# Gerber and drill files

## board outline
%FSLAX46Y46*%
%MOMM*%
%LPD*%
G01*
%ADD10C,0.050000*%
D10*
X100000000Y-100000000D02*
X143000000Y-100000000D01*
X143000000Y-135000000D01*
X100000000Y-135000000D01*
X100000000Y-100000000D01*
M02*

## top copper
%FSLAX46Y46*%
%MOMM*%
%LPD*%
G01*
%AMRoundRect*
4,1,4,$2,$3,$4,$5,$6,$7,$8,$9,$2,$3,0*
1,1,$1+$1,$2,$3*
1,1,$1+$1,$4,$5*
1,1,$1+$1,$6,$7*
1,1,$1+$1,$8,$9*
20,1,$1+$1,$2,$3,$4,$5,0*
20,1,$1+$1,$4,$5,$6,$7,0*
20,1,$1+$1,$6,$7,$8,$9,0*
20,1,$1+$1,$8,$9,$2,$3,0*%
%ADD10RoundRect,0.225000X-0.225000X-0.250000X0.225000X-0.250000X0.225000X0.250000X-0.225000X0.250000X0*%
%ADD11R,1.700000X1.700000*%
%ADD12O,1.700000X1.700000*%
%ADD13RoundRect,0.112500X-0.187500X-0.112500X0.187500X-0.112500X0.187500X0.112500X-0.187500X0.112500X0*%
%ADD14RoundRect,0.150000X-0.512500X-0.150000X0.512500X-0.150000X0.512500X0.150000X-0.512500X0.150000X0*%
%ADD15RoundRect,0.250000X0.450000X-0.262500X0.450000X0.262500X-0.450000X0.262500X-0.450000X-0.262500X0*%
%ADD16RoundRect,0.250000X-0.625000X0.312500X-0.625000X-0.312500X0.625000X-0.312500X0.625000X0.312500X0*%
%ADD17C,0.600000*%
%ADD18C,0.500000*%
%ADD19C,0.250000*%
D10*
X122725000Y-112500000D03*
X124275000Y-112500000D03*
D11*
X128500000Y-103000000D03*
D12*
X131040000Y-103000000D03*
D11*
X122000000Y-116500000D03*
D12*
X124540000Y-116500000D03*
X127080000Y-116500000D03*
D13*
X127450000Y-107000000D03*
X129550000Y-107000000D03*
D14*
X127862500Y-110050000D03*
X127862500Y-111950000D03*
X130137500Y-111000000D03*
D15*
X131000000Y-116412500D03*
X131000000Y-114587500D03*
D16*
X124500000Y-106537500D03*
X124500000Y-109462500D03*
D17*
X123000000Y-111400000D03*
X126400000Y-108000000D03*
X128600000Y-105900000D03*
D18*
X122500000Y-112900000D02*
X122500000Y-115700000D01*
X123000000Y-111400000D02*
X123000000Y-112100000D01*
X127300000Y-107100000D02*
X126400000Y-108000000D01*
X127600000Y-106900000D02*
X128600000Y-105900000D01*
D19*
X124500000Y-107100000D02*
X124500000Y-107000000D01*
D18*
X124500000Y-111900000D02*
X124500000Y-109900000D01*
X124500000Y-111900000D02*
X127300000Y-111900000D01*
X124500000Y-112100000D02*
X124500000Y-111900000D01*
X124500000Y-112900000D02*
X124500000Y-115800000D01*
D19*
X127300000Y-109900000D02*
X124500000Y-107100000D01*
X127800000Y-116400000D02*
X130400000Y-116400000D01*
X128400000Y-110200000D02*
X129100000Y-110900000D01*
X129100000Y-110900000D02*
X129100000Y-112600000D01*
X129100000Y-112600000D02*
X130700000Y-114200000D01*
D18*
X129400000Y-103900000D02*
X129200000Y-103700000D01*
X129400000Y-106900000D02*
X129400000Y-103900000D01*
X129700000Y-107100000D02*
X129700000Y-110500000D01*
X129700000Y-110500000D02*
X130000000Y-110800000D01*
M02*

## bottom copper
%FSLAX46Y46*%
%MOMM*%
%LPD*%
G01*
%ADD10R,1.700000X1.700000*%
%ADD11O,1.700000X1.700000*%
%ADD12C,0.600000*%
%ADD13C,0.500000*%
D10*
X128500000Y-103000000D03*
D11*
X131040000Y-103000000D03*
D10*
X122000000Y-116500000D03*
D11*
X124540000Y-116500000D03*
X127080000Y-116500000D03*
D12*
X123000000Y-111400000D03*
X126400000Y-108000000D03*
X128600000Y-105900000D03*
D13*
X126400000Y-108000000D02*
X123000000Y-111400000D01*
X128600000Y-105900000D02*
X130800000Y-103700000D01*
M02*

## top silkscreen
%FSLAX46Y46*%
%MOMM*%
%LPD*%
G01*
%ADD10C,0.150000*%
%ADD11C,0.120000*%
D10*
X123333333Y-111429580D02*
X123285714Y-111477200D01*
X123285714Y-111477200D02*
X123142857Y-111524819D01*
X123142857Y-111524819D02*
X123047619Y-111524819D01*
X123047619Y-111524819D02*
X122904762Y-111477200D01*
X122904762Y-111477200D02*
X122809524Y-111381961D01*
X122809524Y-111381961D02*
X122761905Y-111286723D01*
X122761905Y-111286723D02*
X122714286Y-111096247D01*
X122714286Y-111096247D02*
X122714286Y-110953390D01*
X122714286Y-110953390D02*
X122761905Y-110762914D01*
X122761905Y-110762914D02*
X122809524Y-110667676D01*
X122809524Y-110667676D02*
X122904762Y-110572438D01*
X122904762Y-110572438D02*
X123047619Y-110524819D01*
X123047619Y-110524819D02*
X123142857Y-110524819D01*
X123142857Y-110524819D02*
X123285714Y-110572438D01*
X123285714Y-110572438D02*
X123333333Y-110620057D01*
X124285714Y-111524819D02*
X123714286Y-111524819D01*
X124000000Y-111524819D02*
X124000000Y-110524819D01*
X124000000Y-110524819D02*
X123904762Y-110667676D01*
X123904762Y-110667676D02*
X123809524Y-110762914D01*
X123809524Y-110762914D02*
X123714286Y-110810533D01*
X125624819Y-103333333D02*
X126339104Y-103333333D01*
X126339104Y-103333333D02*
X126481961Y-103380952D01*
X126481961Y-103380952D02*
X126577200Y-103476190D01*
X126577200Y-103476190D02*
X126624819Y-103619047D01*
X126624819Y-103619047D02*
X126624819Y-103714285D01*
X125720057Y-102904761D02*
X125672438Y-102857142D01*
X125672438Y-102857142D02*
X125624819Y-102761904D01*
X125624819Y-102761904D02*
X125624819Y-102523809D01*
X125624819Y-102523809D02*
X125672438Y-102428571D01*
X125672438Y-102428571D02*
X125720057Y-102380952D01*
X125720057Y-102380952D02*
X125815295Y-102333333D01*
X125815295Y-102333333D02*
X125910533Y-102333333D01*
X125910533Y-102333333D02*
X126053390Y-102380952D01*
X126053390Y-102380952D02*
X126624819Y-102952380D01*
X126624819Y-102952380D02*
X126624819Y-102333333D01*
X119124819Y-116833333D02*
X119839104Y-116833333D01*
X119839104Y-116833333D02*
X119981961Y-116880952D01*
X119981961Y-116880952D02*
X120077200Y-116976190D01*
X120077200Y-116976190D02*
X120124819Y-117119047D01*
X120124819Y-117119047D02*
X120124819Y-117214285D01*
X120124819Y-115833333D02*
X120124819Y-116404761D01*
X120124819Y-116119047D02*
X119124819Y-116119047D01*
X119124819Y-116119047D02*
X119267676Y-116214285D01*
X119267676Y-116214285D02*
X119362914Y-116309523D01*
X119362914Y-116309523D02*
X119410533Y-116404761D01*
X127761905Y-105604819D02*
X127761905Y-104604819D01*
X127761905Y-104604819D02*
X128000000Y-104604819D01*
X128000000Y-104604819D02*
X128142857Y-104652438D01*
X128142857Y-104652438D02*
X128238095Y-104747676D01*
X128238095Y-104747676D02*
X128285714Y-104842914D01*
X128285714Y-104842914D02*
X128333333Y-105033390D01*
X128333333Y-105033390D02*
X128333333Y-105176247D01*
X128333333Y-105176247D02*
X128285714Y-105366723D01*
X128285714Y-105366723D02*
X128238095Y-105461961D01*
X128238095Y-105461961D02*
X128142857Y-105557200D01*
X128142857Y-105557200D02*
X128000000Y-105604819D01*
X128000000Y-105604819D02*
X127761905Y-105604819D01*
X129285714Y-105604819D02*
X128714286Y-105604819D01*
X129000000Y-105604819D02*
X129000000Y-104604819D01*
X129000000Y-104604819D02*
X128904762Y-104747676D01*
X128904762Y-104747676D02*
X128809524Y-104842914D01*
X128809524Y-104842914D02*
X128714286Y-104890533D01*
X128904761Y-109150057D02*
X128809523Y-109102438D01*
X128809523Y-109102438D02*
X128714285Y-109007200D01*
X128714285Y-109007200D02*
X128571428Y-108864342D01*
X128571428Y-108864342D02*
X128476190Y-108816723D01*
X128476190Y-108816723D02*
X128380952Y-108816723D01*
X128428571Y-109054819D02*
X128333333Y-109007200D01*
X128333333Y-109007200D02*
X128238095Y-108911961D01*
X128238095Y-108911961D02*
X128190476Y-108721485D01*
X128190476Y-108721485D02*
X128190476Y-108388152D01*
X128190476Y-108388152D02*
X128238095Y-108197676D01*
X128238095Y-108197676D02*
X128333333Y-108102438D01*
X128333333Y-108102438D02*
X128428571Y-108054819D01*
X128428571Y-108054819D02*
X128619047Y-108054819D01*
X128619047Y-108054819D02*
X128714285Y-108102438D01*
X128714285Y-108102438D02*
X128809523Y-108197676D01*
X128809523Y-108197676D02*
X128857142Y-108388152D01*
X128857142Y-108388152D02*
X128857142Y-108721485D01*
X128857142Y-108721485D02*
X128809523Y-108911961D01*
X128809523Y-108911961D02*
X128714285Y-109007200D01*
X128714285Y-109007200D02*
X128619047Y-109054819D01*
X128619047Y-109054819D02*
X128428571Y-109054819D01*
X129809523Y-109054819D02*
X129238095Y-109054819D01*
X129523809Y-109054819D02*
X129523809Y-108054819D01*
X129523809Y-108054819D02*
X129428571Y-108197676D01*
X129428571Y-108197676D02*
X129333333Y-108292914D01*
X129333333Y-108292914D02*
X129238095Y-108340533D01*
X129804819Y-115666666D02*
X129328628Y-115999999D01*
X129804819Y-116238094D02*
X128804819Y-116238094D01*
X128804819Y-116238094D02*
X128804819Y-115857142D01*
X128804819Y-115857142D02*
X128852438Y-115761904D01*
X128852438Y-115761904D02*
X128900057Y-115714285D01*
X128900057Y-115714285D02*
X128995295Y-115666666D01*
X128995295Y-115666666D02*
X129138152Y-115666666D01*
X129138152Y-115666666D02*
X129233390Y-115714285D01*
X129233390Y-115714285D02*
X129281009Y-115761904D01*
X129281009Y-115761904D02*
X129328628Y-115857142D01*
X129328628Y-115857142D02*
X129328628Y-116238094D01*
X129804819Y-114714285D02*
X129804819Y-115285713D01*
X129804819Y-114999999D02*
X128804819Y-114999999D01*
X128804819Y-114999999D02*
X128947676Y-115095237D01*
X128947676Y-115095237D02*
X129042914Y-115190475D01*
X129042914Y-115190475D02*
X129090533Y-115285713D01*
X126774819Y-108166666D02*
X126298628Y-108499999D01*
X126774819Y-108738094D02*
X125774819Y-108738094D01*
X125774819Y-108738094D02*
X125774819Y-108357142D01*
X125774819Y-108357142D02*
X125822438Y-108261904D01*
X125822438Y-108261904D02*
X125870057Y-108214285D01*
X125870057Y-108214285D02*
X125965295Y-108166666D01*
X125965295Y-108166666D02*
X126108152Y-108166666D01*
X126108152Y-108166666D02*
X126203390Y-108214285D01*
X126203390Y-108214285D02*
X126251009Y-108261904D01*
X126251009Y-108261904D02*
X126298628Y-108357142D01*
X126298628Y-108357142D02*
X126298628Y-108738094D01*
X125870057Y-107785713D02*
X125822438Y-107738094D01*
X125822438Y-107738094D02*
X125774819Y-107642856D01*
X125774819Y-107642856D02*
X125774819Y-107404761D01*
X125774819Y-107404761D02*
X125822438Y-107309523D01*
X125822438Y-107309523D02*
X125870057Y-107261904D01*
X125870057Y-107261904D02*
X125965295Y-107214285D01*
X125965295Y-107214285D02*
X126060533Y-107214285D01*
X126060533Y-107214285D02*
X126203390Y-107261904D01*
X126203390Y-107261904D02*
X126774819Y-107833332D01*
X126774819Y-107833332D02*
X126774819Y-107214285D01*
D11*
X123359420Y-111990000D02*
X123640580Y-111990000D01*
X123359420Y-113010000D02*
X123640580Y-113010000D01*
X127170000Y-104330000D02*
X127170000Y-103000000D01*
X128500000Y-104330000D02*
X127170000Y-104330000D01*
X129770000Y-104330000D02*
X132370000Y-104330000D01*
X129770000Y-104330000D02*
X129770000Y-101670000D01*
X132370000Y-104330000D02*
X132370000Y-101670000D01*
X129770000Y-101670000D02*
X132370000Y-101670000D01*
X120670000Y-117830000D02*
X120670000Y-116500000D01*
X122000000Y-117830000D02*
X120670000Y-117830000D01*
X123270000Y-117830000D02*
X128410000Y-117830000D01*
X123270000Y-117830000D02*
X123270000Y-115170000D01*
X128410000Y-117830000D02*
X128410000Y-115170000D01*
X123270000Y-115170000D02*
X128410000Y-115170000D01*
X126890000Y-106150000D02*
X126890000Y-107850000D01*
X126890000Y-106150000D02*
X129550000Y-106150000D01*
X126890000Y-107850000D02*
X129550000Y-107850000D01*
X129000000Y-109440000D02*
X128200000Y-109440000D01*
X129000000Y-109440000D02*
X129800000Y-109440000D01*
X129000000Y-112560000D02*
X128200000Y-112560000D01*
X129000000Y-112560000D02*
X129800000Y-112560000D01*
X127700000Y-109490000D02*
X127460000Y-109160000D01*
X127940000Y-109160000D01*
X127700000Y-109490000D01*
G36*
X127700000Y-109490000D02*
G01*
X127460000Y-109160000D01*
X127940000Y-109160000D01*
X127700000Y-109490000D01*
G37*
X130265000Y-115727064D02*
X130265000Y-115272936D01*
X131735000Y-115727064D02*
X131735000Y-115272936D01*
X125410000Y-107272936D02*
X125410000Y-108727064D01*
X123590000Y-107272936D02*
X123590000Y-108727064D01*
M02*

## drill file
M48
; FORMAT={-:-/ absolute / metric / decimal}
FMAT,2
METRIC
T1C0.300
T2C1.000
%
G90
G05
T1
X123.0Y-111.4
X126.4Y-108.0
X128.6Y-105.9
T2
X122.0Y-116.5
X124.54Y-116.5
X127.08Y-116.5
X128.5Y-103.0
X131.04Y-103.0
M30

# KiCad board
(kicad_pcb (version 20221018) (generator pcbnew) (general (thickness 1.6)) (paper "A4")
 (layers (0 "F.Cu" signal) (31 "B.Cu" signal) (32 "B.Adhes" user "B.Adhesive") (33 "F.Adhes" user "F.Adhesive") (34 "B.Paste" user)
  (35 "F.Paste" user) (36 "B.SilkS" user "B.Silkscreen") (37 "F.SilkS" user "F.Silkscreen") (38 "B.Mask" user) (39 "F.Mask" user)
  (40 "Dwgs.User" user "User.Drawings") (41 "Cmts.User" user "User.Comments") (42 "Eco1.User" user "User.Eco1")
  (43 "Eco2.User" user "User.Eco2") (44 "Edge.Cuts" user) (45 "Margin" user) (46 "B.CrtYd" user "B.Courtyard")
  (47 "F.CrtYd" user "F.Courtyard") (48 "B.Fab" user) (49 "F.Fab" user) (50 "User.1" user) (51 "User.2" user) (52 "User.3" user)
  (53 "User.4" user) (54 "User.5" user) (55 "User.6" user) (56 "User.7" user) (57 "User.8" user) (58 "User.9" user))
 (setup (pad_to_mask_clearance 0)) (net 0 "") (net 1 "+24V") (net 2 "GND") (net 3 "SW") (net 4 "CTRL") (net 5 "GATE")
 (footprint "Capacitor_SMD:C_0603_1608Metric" (layer "F.Cu") (at 123.5 112.5)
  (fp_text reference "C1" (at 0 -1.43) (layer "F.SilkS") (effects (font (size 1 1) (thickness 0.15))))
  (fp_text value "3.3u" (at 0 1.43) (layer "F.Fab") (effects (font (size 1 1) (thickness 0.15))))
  (fp_line (start -0.14058 -0.51) (end 0.14058 -0.51) (stroke (width 0.12) (type solid)) (layer "F.SilkS"))
  (fp_line (start -0.14058 0.51) (end 0.14058 0.51) (stroke (width 0.12) (type solid)) (layer "F.SilkS"))
  (pad "1" smd roundrect (at -0.775 0) (size 0.9 0.95) (layers "F.Cu" "F.Paste" "F.Mask") (roundrect_rratio 0.25) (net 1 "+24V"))
  (pad "2" smd roundrect (at 0.775 0) (size 0.9 0.95) (layers "F.Cu" "F.Paste" "F.Mask") (roundrect_rratio 0.25) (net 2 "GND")))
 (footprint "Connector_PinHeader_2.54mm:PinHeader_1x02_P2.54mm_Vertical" (layer "F.Cu") (at 128.5 103 90)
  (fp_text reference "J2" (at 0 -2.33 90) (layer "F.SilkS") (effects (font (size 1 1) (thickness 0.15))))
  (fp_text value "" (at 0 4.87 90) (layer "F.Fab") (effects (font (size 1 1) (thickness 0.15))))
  (fp_line (start -1.33 -1.33) (end 0 -1.33) (stroke (width 0.12) (type solid)) (layer "F.SilkS"))
  (fp_line (start -1.33 0) (end -1.33 -1.33) (stroke (width 0.12) (type solid)) (layer "F.SilkS"))
  (fp_line (start -1.33 1.27) (end -1.33 3.87) (stroke (width 0.12) (type solid)) (layer "F.SilkS"))
  (fp_line (start -1.33 1.27) (end 1.33 1.27) (stroke (width 0.12) (type solid)) (layer "F.SilkS"))
  (fp_line (start -1.33 3.87) (end 1.33 3.87) (stroke (width 0.12) (type solid)) (layer "F.SilkS"))
  (fp_line (start 1.33 1.27) (end 1.33 3.87) (stroke (width 0.12) (type solid)) (layer "F.SilkS"))
  (pad "1" thru_hole rect (at 0 0 90) (size 1.7 1.7) (drill 1) (layers "*.Cu" "*.Mask") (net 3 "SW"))
  (pad "2" thru_hole oval (at 0 2.54 90) (size 1.7 1.7) (drill 1) (layers "*.Cu" "*.Mask") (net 1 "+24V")))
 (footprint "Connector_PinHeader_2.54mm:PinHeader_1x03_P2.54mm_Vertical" (layer "F.Cu") (at 122 116.5 90)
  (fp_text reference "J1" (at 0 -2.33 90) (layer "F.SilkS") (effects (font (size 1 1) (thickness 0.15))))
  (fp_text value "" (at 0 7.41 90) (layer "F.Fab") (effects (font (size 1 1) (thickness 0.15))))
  (fp_line (start -1.33 -1.33) (end 0 -1.33) (stroke (width 0.12) (type solid)) (layer "F.SilkS"))
  (fp_line (start -1.33 0) (end -1.33 -1.33) (stroke (width 0.12) (type solid)) (layer "F.SilkS"))
  (fp_line (start -1.33 1.27) (end -1.33 6.41) (stroke (width 0.12) (type solid)) (layer "F.SilkS"))
  (fp_line (start -1.33 1.27) (end 1.33 1.27) (stroke (width 0.12) (type solid)) (layer "F.SilkS"))
  (fp_line (start -1.33 6.41) (end 1.33 6.41) (stroke (width 0.12) (type solid)) (layer "F.SilkS"))
  (fp_line (start 1.33 1.27) (end 1.33 6.41) (stroke (width 0.12) (type solid)) (layer "F.SilkS"))
  (pad "1" thru_hole rect (at 0 0 90) (size 1.7 1.7) (drill 1) (layers "*.Cu" "*.Mask") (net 1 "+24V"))
  (pad "2" thru_hole oval (at 0 2.54 90) (size 1.7 1.7) (drill 1) (layers "*.Cu" "*.Mask") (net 2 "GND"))
  (pad "3" thru_hole oval (at 0 5.08 90) (size 1.7 1.7) (drill 1) (layers "*.Cu" "*.Mask") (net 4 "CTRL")))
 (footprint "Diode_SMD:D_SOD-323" (layer "F.Cu") (at 128.5 107)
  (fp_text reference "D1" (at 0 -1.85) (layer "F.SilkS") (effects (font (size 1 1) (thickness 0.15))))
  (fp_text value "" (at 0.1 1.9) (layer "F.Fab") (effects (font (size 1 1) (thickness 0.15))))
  (fp_line (start -1.61 -0.85) (end -1.61 0.85) (stroke (width 0.12) (type solid)) (layer "F.SilkS"))
  (fp_line (start -1.61 -0.85) (end 1.05 -0.85) (stroke (width 0.12) (type solid)) (layer "F.SilkS"))
  (fp_line (start -1.61 0.85) (end 1.05 0.85) (stroke (width 0.12) (type solid)) (layer "F.SilkS"))
  (pad "1" smd roundrect (at -1.05 0) (size 0.6 0.45) (layers "F.Cu" "F.Paste" "F.Mask") (roundrect_rratio 0.25) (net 1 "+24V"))
  (pad "2" smd roundrect (at 1.05 0) (size 0.6 0.45) (layers "F.Cu" "F.Paste" "F.Mask") (roundrect_rratio 0.25) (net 3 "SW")))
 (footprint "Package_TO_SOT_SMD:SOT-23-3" (layer "F.Cu") (at 129 111)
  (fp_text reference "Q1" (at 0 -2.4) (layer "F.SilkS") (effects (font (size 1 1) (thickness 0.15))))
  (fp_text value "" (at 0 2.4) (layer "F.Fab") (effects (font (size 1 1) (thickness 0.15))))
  (fp_line (start 0 -1.56) (end -0.8 -1.56) (stroke (width 0.12) (type solid)) (layer "F.SilkS"))
  (fp_line (start 0 -1.56) (end 0.8 -1.56) (stroke (width 0.12) (type solid)) (layer "F.SilkS"))
  (fp_line (start 0 1.56) (end -0.8 1.56) (stroke (width 0.12) (type solid)) (layer "F.SilkS"))
  (fp_line (start 0 1.56) (end 0.8 1.56) (stroke (width 0.12) (type solid)) (layer "F.SilkS"))
  (fp_poly
   (pts (xy -1.3 -1.51) (xy -1.54 -1.84) (xy -1.06 -1.84) (xy -1.3 -1.51)) (stroke (width 0.12) (type solid)) (fill solid) (layer "F.SilkS"))
  (pad "1" smd roundrect (at -1.1375 -0.95) (size 1.325 0.6) (layers "F.Cu" "F.Paste" "F.Mask") (roundrect_rratio 0.25) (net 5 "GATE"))
  (pad "2" smd roundrect (at -1.1375 0.95) (size 1.325 0.6) (layers "F.Cu" "F.Paste" "F.Mask") (roundrect_rratio 0.25) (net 2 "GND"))
  (pad "3" smd roundrect (at 1.1375 0) (size 1.325 0.6) (layers "F.Cu" "F.Paste" "F.Mask") (roundrect_rratio 0.25) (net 3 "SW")))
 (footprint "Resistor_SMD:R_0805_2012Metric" (layer "F.Cu") (at 131 115.5 90)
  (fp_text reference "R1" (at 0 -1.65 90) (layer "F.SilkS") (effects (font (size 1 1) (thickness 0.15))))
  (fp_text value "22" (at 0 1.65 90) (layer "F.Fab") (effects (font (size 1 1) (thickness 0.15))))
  (fp_line (start -0.227064 -0.735) (end 0.227064 -0.735) (stroke (width 0.12) (type solid)) (layer "F.SilkS"))
  (fp_line (start -0.227064 0.735) (end 0.227064 0.735) (stroke (width 0.12) (type solid)) (layer "F.SilkS"))
  (pad "1" smd roundrect (at -0.9125 0 90) (size 1.025 1.4) (layers "F.Cu" "F.Paste" "F.Mask") (roundrect_rratio 0.243902) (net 4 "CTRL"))
  (pad "2" smd roundrect (at 0.9125 0 90) (size 1.025 1.4) (layers "F.Cu" "F.Paste" "F.Mask") (roundrect_rratio 0.243902) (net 5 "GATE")))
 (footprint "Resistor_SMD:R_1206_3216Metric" (layer "F.Cu") (at 124.5 108 -90)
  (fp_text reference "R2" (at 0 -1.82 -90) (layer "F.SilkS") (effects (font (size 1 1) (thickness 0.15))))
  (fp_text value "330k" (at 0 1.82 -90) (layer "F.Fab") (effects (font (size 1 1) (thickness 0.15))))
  (fp_line (start -0.727064 -0.91) (end 0.727064 -0.91) (stroke (width 0.12) (type solid)) (layer "F.SilkS"))
  (fp_line (start -0.727064 0.91) (end 0.727064 0.91) (stroke (width 0.12) (type solid)) (layer "F.SilkS"))
  (pad "1" smd roundrect (at -1.4625 0 270) (size 1.125 1.75) (layers "F.Cu" "F.Paste" "F.Mask") (roundrect_rratio 0.222222) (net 5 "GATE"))
  (pad "2" smd roundrect (at 1.4625 0 270) (size 1.125 1.75) (layers "F.Cu" "F.Paste" "F.Mask") (roundrect_rratio 0.222222) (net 2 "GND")))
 (gr_rect (start 100 100) (end 143 135) (stroke (width 0.05) (type default)) (fill none) (layer "Edge.Cuts"))
 (segment (start 122.5 112.9) (end 122.5 115.7) (width 0.5) (layer "F.Cu") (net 1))
 (segment (start 123 111.4) (end 123 112.1) (width 0.5) (layer "F.Cu") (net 1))
 (segment (start 127.3 107.1) (end 126.4 108) (width 0.5) (layer "F.Cu") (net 1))
 (segment (start 127.6 106.9) (end 128.6 105.9) (width 0.5) (layer "F.Cu") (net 1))
 (via (at 123 111.4) (size 0.6) (drill 0.3) (layers "F.Cu" "B.Cu") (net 1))
 (via (at 126.4 108) (size 0.6) (drill 0.3) (layers "F.Cu" "B.Cu") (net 1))
 (via (at 128.6 105.9) (size 0.6) (drill 0.3) (layers "F.Cu" "B.Cu") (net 1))
 (segment (start 124.5 107.1) (end 124.5 107) (width 0.25) (layer "F.Cu") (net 5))
 (segment (start 124.5 111.9) (end 124.5 109.9) (width 0.5) (layer "F.Cu") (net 2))
 (segment (start 124.5 111.9) (end 127.3 111.9) (width 0.5) (layer "F.Cu") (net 2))
 (segment (start 124.5 112.1) (end 124.5 111.9) (width 0.5) (layer "F.Cu") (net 2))
 (segment (start 124.5 112.9) (end 124.5 115.8) (width 0.5) (layer "F.Cu") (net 2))
 (segment (start 126.4 108) (end 123 111.4) (width 0.5) (layer "B.Cu") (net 1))
 (segment (start 127.3 109.9) (end 124.5 107.1) (width 0.25) (layer "F.Cu") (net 5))
 (segment (start 127.8 116.4) (end 130.4 116.4) (width 0.25) (layer "F.Cu") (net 4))
 (segment (start 128.4 110.2) (end 129.1 110.9) (width 0.25) (layer "F.Cu") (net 5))
 (segment (start 128.6 105.9) (end 130.8 103.7) (width 0.5) (layer "B.Cu") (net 1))
 (segment (start 129.1 110.9) (end 129.1 112.6) (width 0.25) (layer "F.Cu") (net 5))
 (segment (start 129.1 112.6) (end 130.7 114.2) (width 0.25) (layer "F.Cu") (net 5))
 (segment (start 129.4 103.9) (end 129.2 103.7) (width 0.5) (layer "F.Cu") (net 3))
 (segment (start 129.4 106.9) (end 129.4 103.9) (width 0.5) (layer "F.Cu") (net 3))
 (segment (start 129.7 107.1) (end 129.7 110.5) (width 0.5) (layer "F.Cu") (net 3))
 (segment (start 129.7 110.5) (end 130 110.8) (width 0.5) (layer "F.Cu") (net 3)))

